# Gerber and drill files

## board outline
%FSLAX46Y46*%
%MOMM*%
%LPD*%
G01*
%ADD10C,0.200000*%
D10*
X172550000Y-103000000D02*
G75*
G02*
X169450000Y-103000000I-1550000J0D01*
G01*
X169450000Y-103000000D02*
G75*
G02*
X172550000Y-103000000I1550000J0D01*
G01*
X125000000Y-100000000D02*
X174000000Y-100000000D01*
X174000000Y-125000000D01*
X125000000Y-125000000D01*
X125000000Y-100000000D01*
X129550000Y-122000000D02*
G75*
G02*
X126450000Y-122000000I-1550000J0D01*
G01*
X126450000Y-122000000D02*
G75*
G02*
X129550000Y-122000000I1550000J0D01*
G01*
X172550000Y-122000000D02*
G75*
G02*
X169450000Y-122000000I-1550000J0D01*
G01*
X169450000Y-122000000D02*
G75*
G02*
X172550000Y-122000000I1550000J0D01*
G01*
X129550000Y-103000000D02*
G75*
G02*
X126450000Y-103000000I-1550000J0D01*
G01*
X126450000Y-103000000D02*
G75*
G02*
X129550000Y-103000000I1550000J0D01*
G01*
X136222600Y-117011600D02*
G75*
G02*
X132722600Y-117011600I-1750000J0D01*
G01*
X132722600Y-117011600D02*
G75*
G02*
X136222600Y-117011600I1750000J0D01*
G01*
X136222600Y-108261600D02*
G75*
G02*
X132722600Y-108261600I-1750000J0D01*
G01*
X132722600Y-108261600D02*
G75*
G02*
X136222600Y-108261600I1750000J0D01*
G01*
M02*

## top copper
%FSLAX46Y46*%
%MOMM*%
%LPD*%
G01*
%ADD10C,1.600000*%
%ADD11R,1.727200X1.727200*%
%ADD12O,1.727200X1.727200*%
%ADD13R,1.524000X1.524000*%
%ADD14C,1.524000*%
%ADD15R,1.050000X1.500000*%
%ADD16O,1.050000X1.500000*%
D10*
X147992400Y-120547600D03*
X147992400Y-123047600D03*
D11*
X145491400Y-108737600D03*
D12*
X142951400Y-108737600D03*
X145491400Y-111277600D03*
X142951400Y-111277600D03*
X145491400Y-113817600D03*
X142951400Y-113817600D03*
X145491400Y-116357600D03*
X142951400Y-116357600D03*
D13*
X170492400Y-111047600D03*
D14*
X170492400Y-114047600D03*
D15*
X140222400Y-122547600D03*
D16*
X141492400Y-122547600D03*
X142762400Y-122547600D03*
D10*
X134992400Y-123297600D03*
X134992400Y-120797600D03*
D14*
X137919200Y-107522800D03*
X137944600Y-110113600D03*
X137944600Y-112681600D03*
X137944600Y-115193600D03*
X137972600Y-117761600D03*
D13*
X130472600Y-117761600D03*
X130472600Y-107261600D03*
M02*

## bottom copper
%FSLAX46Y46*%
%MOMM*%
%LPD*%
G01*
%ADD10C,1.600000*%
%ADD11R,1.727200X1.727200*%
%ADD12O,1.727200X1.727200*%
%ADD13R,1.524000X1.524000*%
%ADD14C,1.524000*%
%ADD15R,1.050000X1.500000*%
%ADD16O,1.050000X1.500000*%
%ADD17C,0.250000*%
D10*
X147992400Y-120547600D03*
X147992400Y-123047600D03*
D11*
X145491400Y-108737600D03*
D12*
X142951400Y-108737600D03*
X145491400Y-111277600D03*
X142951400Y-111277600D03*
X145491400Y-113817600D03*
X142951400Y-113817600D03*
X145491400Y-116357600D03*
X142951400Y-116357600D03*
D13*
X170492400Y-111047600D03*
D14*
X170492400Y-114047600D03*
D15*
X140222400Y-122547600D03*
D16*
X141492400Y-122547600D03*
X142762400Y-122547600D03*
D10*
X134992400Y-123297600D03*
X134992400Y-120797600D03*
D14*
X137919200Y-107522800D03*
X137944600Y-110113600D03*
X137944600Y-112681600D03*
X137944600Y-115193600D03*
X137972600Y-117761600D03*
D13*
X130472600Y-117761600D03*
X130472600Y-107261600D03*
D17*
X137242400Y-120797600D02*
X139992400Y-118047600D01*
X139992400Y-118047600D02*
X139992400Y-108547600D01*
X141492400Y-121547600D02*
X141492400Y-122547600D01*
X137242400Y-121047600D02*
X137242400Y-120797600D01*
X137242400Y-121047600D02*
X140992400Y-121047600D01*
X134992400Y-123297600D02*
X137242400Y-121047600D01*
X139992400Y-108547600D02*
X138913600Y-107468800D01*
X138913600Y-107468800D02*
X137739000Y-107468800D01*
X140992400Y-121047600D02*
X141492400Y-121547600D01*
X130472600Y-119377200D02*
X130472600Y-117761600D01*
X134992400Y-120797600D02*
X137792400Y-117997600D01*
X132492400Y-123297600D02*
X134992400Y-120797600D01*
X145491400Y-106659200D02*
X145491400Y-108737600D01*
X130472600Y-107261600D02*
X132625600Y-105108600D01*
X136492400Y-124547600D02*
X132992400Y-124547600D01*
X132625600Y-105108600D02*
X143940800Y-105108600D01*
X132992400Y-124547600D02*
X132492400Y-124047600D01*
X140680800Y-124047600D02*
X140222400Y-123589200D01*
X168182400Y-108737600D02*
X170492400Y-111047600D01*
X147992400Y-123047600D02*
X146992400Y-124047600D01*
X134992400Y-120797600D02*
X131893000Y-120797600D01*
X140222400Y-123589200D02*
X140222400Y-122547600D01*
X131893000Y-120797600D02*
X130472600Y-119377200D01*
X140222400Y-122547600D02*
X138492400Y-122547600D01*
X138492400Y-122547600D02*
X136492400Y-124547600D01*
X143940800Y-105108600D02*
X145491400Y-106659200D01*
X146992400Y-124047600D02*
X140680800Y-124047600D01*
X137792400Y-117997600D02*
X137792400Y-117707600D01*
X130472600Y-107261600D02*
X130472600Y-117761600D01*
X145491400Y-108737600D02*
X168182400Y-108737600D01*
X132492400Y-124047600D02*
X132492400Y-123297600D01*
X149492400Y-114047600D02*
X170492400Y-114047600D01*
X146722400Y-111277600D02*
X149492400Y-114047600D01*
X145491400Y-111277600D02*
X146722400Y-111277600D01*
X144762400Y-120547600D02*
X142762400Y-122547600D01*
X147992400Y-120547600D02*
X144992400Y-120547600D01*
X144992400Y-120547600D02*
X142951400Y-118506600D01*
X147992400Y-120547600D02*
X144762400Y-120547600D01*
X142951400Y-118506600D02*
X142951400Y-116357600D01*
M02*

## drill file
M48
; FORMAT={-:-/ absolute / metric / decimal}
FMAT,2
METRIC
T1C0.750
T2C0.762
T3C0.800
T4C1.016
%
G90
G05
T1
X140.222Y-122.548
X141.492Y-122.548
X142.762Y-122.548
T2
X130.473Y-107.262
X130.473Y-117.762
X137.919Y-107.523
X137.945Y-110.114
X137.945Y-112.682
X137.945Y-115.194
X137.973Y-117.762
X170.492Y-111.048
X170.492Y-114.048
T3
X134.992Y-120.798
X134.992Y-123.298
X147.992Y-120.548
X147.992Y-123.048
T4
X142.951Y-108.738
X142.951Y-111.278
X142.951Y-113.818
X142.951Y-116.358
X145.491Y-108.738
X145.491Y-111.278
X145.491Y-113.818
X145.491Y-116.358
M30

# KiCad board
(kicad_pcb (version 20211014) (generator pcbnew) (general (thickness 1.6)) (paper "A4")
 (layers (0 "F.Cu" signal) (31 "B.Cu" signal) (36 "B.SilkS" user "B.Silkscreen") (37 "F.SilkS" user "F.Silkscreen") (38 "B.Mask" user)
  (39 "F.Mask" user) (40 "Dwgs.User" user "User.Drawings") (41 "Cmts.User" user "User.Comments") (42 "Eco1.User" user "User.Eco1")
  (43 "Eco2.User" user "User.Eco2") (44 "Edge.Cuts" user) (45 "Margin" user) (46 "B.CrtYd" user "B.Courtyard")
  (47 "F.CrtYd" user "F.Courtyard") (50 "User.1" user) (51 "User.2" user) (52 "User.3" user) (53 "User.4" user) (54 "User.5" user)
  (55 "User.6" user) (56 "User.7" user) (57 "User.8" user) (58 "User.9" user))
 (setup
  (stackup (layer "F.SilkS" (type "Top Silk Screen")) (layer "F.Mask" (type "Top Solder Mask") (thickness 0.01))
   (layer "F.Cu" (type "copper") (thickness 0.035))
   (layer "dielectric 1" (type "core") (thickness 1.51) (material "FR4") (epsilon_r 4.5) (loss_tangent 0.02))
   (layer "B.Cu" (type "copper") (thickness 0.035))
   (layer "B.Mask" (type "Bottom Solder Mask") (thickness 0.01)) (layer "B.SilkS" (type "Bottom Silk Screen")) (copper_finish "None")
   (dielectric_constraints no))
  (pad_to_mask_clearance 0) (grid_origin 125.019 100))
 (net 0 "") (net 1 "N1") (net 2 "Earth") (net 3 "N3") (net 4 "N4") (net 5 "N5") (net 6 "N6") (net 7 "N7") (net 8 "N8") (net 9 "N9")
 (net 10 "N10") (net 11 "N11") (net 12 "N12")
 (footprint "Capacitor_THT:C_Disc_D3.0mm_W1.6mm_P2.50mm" (layer "F.Cu") (at 147.9924 120.5476 -90)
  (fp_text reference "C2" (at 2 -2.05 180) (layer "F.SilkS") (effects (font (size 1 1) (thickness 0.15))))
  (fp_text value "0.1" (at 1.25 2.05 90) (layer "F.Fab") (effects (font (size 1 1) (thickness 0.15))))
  (pad "1" thru_hole circle (at 0 0 270) (size 1.6 1.6) (drill 0.8) (layers *.Cu *.Mask) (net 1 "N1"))
  (pad "2" thru_hole circle (at 2.5 0 270) (size 1.6 1.6) (drill 0.8) (layers *.Cu *.Mask) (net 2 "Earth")))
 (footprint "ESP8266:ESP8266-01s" (layer "F.Cu") (at 142.9514 108.7376)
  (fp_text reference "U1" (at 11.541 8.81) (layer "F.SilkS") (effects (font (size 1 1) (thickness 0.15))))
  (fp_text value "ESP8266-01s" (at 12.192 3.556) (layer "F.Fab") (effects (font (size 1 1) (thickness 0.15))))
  (pad "1" thru_hole rect (at 2.54 0) (size 1.7272 1.7272) (drill 1.016) (layers *.Cu *.Mask) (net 2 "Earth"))
  (pad "2" thru_hole oval (at 0 0) (size 1.7272 1.7272) (drill 1.016) (layers *.Cu *.Mask) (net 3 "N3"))
  (pad "3" thru_hole oval (at 2.54 2.54) (size 1.7272 1.7272) (drill 1.016) (layers *.Cu *.Mask) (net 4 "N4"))
  (pad "4" thru_hole oval (at 0 2.54) (size 1.7272 1.7272) (drill 1.016) (layers *.Cu *.Mask) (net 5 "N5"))
  (pad "5" thru_hole oval (at 2.54 5.08) (size 1.7272 1.7272) (drill 1.016) (layers *.Cu *.Mask) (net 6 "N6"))
  (pad "6" thru_hole oval (at 0 5.08) (size 1.7272 1.7272) (drill 1.016) (layers *.Cu *.Mask) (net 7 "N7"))
  (pad "7" thru_hole oval (at 2.54 7.62) (size 1.7272 1.7272) (drill 1.016) (layers *.Cu *.Mask) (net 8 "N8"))
  (pad "8" thru_hole oval (at 0 7.62) (size 1.7272 1.7272) (drill 1.016) (layers *.Cu *.Mask) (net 1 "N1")))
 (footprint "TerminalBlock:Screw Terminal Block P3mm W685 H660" (layer "F.Cu") (at 170.4924 111.0476 -90)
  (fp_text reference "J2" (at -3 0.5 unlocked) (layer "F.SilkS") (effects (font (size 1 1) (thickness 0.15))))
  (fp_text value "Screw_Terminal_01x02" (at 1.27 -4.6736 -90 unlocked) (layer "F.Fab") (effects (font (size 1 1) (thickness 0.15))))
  (pad "1" thru_hole rect (at 0 0 270) (size 1.524 1.524) (drill 0.762) (layers *.Cu *.Mask) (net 2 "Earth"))
  (pad "2" thru_hole circle (at 3 0 270) (size 1.524 1.524) (drill 0.762) (layers *.Cu *.Mask) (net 4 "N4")))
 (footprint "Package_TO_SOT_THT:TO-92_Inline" (layer "F.Cu") (at 140.2224 122.5476)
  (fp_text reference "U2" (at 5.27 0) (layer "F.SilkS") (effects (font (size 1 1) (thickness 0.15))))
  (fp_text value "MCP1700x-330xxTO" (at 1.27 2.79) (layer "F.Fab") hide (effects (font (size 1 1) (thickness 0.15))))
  (pad "1" thru_hole rect (at 0 0) (size 1.05 1.5) (drill 0.75) (layers *.Cu *.Mask) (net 2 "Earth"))
  (pad "2" thru_hole oval (at 1.27 0) (size 1.05 1.5) (drill 0.75) (layers *.Cu *.Mask) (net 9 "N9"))
  (pad "3" thru_hole oval (at 2.54 0) (size 1.05 1.5) (drill 0.75) (layers *.Cu *.Mask) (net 1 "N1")))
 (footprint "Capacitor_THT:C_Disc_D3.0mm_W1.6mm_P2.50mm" (layer "F.Cu") (at 134.9924 123.2976 90)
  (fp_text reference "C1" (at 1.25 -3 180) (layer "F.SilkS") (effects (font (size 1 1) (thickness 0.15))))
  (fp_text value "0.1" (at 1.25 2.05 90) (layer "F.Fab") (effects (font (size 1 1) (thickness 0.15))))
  (pad "1" thru_hole circle (at 0 0 90) (size 1.6 1.6) (drill 0.8) (layers *.Cu *.Mask) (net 9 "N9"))
  (pad "2" thru_hole circle (at 2.5 0 90) (size 1.6 1.6) (drill 0.8) (layers *.Cu *.Mask) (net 2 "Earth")))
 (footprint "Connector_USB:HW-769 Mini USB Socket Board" (layer "F.Cu") (at 139.7226 119.5116)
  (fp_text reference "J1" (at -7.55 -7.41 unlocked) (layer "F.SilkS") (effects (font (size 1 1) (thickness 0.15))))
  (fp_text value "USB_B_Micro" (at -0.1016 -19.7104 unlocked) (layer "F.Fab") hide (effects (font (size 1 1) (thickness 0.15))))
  (fp_circle (center -5.25 -2.5) (end -3.5 -2.5) (layer "Edge.Cuts") (width 0.2) (fill none))
  (fp_circle (center -5.25 -11.25) (end -3.5 -11.25) (layer "Edge.Cuts") (width 0.2) (fill none))
  (pad "1" thru_hole circle (at -1.8034 -11.9888) (size 1.524 1.524) (drill 0.762) (layers *.Cu *.Mask) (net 9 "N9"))
  (pad "2" thru_hole circle (at -1.778 -9.398) (size 1.524 1.524) (drill 0.762) (layers *.Cu *.Mask) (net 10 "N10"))
  (pad "3" thru_hole circle (at -1.778 -6.83) (size 1.524 1.524) (drill 0.762) (layers *.Cu *.Mask) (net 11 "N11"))
  (pad "4" thru_hole circle (at -1.778 -4.318) (size 1.524 1.524) (drill 0.762) (layers *.Cu *.Mask) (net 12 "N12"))
  (pad "5" thru_hole circle (at -1.75 -1.75) (size 1.524 1.524) (drill 0.762) (layers *.Cu *.Mask) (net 2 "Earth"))
  (pad "6" thru_hole rect (at -9.25 -1.75) (size 1.524 1.524) (drill 0.762) (layers *.Cu *.Mask) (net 2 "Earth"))
  (pad "7" thru_hole rect (at -9.25 -12.25) (size 1.524 1.524) (drill 0.762) (layers *.Cu *.Mask) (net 2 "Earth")))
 (gr_circle (center 171 103) (end 172.55 103) (layer "Edge.Cuts") (width 0.2) (fill none))
 (gr_rect (start 125 100) (end 174 125) (layer "Edge.Cuts") (width 0.2) (fill none))
 (gr_circle (center 128 122) (end 129.55 122) (layer "Edge.Cuts") (width 0.2) (fill none))
 (gr_circle (center 171 122) (end 172.55 122) (layer "Edge.Cuts") (width 0.2) (fill none))
 (gr_circle (center 128 103) (end 129.55 103) (layer "Edge.Cuts") (width 0.2) (fill none))
 (segment (start 137.2424 120.7976) (end 139.9924 118.0476) (width 0.25) (layer "B.Cu") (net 9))
 (segment (start 139.9924 118.0476) (end 139.9924 108.5476) (width 0.25) (layer "B.Cu") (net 9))
 (segment (start 141.4924 121.5476) (end 141.4924 122.5476) (width 0.25) (layer "B.Cu") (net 9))
 (segment (start 137.2424 121.0476) (end 137.2424 120.7976) (width 0.25) (layer "B.Cu") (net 9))
 (segment (start 137.2424 121.0476) (end 140.9924 121.0476) (width 0.25) (layer "B.Cu") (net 9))
 (segment (start 134.9924 123.2976) (end 137.2424 121.0476) (width 0.25) (layer "B.Cu") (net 9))
 (segment (start 139.9924 108.5476) (end 138.9136 107.4688) (width 0.25) (layer "B.Cu") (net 9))
 (segment (start 138.9136 107.4688) (end 137.739 107.4688) (width 0.25) (layer "B.Cu") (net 9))
 (segment (start 140.9924 121.0476) (end 141.4924 121.5476) (width 0.25) (layer "B.Cu") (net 9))
 (segment (start 130.4726 119.3772) (end 130.4726 117.7616) (width 0.25) (layer "B.Cu") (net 2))
 (segment (start 134.9924 120.7976) (end 137.7924 117.9976) (width 0.25) (layer "B.Cu") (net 2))
 (segment (start 132.4924 123.2976) (end 134.9924 120.7976) (width 0.25) (layer "B.Cu") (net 2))
 (segment (start 145.4914 106.6592) (end 145.4914 108.7376) (width 0.25) (layer "B.Cu") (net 2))
 (segment (start 130.4726 107.2616) (end 132.6256 105.1086) (width 0.25) (layer "B.Cu") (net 2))
 (segment (start 136.4924 124.5476) (end 132.9924 124.5476) (width 0.25) (layer "B.Cu") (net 2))
 (segment (start 132.6256 105.1086) (end 143.9408 105.1086) (width 0.25) (layer "B.Cu") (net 2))
 (segment (start 132.9924 124.5476) (end 132.4924 124.0476) (width 0.25) (layer "B.Cu") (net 2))
 (segment (start 140.6808 124.0476) (end 140.2224 123.5892) (width 0.25) (layer "B.Cu") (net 2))
 (segment (start 168.1824 108.7376) (end 170.4924 111.0476) (width 0.25) (layer "B.Cu") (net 2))
 (segment (start 147.9924 123.0476) (end 146.9924 124.0476) (width 0.25) (layer "B.Cu") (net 2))
 (segment (start 134.9924 120.7976) (end 131.893 120.7976) (width 0.25) (layer "B.Cu") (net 2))
 (segment (start 140.2224 123.5892) (end 140.2224 122.5476) (width 0.25) (layer "B.Cu") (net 2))
 (segment (start 131.893 120.7976) (end 130.4726 119.3772) (width 0.25) (layer "B.Cu") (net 2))
 (segment (start 140.2224 122.5476) (end 138.4924 122.5476) (width 0.25) (layer "B.Cu") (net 2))
 (segment (start 138.4924 122.5476) (end 136.4924 124.5476) (width 0.25) (layer "B.Cu") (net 2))
 (segment (start 143.9408 105.1086) (end 145.4914 106.6592) (width 0.25) (layer "B.Cu") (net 2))
 (segment (start 146.9924 124.0476) (end 140.6808 124.0476) (width 0.25) (layer "B.Cu") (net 2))
 (segment (start 137.7924 117.9976) (end 137.7924 117.7076) (width 0.25) (layer "B.Cu") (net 2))
 (segment (start 130.4726 107.2616) (end 130.4726 117.7616) (width 0.25) (layer "B.Cu") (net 2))
 (segment (start 145.4914 108.7376) (end 168.1824 108.7376) (width 0.25) (layer "B.Cu") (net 2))
 (segment (start 132.4924 124.0476) (end 132.4924 123.2976) (width 0.25) (layer "B.Cu") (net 2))
 (segment (start 149.4924 114.0476) (end 170.4924 114.0476) (width 0.25) (layer "B.Cu") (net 4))
 (segment (start 146.7224 111.2776) (end 149.4924 114.0476) (width 0.25) (layer "B.Cu") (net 4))
 (segment (start 145.4914 111.2776) (end 146.7224 111.2776) (width 0.25) (layer "B.Cu") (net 4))
 (segment (start 144.7624 120.5476) (end 142.7624 122.5476) (width 0.25) (layer "B.Cu") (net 1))
 (segment (start 147.9924 120.5476) (end 144.9924 120.5476) (width 0.25) (layer "B.Cu") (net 1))
 (segment (start 144.9924 120.5476) (end 142.9514 118.5066) (width 0.25) (layer "B.Cu") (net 1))
 (segment (start 147.9924 120.5476) (end 144.7624 120.5476) (width 0.25) (layer "B.Cu") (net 1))
 (segment (start 142.9514 118.5066) (end 142.9514 116.3576) (width 0.25) (layer "B.Cu") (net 1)))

